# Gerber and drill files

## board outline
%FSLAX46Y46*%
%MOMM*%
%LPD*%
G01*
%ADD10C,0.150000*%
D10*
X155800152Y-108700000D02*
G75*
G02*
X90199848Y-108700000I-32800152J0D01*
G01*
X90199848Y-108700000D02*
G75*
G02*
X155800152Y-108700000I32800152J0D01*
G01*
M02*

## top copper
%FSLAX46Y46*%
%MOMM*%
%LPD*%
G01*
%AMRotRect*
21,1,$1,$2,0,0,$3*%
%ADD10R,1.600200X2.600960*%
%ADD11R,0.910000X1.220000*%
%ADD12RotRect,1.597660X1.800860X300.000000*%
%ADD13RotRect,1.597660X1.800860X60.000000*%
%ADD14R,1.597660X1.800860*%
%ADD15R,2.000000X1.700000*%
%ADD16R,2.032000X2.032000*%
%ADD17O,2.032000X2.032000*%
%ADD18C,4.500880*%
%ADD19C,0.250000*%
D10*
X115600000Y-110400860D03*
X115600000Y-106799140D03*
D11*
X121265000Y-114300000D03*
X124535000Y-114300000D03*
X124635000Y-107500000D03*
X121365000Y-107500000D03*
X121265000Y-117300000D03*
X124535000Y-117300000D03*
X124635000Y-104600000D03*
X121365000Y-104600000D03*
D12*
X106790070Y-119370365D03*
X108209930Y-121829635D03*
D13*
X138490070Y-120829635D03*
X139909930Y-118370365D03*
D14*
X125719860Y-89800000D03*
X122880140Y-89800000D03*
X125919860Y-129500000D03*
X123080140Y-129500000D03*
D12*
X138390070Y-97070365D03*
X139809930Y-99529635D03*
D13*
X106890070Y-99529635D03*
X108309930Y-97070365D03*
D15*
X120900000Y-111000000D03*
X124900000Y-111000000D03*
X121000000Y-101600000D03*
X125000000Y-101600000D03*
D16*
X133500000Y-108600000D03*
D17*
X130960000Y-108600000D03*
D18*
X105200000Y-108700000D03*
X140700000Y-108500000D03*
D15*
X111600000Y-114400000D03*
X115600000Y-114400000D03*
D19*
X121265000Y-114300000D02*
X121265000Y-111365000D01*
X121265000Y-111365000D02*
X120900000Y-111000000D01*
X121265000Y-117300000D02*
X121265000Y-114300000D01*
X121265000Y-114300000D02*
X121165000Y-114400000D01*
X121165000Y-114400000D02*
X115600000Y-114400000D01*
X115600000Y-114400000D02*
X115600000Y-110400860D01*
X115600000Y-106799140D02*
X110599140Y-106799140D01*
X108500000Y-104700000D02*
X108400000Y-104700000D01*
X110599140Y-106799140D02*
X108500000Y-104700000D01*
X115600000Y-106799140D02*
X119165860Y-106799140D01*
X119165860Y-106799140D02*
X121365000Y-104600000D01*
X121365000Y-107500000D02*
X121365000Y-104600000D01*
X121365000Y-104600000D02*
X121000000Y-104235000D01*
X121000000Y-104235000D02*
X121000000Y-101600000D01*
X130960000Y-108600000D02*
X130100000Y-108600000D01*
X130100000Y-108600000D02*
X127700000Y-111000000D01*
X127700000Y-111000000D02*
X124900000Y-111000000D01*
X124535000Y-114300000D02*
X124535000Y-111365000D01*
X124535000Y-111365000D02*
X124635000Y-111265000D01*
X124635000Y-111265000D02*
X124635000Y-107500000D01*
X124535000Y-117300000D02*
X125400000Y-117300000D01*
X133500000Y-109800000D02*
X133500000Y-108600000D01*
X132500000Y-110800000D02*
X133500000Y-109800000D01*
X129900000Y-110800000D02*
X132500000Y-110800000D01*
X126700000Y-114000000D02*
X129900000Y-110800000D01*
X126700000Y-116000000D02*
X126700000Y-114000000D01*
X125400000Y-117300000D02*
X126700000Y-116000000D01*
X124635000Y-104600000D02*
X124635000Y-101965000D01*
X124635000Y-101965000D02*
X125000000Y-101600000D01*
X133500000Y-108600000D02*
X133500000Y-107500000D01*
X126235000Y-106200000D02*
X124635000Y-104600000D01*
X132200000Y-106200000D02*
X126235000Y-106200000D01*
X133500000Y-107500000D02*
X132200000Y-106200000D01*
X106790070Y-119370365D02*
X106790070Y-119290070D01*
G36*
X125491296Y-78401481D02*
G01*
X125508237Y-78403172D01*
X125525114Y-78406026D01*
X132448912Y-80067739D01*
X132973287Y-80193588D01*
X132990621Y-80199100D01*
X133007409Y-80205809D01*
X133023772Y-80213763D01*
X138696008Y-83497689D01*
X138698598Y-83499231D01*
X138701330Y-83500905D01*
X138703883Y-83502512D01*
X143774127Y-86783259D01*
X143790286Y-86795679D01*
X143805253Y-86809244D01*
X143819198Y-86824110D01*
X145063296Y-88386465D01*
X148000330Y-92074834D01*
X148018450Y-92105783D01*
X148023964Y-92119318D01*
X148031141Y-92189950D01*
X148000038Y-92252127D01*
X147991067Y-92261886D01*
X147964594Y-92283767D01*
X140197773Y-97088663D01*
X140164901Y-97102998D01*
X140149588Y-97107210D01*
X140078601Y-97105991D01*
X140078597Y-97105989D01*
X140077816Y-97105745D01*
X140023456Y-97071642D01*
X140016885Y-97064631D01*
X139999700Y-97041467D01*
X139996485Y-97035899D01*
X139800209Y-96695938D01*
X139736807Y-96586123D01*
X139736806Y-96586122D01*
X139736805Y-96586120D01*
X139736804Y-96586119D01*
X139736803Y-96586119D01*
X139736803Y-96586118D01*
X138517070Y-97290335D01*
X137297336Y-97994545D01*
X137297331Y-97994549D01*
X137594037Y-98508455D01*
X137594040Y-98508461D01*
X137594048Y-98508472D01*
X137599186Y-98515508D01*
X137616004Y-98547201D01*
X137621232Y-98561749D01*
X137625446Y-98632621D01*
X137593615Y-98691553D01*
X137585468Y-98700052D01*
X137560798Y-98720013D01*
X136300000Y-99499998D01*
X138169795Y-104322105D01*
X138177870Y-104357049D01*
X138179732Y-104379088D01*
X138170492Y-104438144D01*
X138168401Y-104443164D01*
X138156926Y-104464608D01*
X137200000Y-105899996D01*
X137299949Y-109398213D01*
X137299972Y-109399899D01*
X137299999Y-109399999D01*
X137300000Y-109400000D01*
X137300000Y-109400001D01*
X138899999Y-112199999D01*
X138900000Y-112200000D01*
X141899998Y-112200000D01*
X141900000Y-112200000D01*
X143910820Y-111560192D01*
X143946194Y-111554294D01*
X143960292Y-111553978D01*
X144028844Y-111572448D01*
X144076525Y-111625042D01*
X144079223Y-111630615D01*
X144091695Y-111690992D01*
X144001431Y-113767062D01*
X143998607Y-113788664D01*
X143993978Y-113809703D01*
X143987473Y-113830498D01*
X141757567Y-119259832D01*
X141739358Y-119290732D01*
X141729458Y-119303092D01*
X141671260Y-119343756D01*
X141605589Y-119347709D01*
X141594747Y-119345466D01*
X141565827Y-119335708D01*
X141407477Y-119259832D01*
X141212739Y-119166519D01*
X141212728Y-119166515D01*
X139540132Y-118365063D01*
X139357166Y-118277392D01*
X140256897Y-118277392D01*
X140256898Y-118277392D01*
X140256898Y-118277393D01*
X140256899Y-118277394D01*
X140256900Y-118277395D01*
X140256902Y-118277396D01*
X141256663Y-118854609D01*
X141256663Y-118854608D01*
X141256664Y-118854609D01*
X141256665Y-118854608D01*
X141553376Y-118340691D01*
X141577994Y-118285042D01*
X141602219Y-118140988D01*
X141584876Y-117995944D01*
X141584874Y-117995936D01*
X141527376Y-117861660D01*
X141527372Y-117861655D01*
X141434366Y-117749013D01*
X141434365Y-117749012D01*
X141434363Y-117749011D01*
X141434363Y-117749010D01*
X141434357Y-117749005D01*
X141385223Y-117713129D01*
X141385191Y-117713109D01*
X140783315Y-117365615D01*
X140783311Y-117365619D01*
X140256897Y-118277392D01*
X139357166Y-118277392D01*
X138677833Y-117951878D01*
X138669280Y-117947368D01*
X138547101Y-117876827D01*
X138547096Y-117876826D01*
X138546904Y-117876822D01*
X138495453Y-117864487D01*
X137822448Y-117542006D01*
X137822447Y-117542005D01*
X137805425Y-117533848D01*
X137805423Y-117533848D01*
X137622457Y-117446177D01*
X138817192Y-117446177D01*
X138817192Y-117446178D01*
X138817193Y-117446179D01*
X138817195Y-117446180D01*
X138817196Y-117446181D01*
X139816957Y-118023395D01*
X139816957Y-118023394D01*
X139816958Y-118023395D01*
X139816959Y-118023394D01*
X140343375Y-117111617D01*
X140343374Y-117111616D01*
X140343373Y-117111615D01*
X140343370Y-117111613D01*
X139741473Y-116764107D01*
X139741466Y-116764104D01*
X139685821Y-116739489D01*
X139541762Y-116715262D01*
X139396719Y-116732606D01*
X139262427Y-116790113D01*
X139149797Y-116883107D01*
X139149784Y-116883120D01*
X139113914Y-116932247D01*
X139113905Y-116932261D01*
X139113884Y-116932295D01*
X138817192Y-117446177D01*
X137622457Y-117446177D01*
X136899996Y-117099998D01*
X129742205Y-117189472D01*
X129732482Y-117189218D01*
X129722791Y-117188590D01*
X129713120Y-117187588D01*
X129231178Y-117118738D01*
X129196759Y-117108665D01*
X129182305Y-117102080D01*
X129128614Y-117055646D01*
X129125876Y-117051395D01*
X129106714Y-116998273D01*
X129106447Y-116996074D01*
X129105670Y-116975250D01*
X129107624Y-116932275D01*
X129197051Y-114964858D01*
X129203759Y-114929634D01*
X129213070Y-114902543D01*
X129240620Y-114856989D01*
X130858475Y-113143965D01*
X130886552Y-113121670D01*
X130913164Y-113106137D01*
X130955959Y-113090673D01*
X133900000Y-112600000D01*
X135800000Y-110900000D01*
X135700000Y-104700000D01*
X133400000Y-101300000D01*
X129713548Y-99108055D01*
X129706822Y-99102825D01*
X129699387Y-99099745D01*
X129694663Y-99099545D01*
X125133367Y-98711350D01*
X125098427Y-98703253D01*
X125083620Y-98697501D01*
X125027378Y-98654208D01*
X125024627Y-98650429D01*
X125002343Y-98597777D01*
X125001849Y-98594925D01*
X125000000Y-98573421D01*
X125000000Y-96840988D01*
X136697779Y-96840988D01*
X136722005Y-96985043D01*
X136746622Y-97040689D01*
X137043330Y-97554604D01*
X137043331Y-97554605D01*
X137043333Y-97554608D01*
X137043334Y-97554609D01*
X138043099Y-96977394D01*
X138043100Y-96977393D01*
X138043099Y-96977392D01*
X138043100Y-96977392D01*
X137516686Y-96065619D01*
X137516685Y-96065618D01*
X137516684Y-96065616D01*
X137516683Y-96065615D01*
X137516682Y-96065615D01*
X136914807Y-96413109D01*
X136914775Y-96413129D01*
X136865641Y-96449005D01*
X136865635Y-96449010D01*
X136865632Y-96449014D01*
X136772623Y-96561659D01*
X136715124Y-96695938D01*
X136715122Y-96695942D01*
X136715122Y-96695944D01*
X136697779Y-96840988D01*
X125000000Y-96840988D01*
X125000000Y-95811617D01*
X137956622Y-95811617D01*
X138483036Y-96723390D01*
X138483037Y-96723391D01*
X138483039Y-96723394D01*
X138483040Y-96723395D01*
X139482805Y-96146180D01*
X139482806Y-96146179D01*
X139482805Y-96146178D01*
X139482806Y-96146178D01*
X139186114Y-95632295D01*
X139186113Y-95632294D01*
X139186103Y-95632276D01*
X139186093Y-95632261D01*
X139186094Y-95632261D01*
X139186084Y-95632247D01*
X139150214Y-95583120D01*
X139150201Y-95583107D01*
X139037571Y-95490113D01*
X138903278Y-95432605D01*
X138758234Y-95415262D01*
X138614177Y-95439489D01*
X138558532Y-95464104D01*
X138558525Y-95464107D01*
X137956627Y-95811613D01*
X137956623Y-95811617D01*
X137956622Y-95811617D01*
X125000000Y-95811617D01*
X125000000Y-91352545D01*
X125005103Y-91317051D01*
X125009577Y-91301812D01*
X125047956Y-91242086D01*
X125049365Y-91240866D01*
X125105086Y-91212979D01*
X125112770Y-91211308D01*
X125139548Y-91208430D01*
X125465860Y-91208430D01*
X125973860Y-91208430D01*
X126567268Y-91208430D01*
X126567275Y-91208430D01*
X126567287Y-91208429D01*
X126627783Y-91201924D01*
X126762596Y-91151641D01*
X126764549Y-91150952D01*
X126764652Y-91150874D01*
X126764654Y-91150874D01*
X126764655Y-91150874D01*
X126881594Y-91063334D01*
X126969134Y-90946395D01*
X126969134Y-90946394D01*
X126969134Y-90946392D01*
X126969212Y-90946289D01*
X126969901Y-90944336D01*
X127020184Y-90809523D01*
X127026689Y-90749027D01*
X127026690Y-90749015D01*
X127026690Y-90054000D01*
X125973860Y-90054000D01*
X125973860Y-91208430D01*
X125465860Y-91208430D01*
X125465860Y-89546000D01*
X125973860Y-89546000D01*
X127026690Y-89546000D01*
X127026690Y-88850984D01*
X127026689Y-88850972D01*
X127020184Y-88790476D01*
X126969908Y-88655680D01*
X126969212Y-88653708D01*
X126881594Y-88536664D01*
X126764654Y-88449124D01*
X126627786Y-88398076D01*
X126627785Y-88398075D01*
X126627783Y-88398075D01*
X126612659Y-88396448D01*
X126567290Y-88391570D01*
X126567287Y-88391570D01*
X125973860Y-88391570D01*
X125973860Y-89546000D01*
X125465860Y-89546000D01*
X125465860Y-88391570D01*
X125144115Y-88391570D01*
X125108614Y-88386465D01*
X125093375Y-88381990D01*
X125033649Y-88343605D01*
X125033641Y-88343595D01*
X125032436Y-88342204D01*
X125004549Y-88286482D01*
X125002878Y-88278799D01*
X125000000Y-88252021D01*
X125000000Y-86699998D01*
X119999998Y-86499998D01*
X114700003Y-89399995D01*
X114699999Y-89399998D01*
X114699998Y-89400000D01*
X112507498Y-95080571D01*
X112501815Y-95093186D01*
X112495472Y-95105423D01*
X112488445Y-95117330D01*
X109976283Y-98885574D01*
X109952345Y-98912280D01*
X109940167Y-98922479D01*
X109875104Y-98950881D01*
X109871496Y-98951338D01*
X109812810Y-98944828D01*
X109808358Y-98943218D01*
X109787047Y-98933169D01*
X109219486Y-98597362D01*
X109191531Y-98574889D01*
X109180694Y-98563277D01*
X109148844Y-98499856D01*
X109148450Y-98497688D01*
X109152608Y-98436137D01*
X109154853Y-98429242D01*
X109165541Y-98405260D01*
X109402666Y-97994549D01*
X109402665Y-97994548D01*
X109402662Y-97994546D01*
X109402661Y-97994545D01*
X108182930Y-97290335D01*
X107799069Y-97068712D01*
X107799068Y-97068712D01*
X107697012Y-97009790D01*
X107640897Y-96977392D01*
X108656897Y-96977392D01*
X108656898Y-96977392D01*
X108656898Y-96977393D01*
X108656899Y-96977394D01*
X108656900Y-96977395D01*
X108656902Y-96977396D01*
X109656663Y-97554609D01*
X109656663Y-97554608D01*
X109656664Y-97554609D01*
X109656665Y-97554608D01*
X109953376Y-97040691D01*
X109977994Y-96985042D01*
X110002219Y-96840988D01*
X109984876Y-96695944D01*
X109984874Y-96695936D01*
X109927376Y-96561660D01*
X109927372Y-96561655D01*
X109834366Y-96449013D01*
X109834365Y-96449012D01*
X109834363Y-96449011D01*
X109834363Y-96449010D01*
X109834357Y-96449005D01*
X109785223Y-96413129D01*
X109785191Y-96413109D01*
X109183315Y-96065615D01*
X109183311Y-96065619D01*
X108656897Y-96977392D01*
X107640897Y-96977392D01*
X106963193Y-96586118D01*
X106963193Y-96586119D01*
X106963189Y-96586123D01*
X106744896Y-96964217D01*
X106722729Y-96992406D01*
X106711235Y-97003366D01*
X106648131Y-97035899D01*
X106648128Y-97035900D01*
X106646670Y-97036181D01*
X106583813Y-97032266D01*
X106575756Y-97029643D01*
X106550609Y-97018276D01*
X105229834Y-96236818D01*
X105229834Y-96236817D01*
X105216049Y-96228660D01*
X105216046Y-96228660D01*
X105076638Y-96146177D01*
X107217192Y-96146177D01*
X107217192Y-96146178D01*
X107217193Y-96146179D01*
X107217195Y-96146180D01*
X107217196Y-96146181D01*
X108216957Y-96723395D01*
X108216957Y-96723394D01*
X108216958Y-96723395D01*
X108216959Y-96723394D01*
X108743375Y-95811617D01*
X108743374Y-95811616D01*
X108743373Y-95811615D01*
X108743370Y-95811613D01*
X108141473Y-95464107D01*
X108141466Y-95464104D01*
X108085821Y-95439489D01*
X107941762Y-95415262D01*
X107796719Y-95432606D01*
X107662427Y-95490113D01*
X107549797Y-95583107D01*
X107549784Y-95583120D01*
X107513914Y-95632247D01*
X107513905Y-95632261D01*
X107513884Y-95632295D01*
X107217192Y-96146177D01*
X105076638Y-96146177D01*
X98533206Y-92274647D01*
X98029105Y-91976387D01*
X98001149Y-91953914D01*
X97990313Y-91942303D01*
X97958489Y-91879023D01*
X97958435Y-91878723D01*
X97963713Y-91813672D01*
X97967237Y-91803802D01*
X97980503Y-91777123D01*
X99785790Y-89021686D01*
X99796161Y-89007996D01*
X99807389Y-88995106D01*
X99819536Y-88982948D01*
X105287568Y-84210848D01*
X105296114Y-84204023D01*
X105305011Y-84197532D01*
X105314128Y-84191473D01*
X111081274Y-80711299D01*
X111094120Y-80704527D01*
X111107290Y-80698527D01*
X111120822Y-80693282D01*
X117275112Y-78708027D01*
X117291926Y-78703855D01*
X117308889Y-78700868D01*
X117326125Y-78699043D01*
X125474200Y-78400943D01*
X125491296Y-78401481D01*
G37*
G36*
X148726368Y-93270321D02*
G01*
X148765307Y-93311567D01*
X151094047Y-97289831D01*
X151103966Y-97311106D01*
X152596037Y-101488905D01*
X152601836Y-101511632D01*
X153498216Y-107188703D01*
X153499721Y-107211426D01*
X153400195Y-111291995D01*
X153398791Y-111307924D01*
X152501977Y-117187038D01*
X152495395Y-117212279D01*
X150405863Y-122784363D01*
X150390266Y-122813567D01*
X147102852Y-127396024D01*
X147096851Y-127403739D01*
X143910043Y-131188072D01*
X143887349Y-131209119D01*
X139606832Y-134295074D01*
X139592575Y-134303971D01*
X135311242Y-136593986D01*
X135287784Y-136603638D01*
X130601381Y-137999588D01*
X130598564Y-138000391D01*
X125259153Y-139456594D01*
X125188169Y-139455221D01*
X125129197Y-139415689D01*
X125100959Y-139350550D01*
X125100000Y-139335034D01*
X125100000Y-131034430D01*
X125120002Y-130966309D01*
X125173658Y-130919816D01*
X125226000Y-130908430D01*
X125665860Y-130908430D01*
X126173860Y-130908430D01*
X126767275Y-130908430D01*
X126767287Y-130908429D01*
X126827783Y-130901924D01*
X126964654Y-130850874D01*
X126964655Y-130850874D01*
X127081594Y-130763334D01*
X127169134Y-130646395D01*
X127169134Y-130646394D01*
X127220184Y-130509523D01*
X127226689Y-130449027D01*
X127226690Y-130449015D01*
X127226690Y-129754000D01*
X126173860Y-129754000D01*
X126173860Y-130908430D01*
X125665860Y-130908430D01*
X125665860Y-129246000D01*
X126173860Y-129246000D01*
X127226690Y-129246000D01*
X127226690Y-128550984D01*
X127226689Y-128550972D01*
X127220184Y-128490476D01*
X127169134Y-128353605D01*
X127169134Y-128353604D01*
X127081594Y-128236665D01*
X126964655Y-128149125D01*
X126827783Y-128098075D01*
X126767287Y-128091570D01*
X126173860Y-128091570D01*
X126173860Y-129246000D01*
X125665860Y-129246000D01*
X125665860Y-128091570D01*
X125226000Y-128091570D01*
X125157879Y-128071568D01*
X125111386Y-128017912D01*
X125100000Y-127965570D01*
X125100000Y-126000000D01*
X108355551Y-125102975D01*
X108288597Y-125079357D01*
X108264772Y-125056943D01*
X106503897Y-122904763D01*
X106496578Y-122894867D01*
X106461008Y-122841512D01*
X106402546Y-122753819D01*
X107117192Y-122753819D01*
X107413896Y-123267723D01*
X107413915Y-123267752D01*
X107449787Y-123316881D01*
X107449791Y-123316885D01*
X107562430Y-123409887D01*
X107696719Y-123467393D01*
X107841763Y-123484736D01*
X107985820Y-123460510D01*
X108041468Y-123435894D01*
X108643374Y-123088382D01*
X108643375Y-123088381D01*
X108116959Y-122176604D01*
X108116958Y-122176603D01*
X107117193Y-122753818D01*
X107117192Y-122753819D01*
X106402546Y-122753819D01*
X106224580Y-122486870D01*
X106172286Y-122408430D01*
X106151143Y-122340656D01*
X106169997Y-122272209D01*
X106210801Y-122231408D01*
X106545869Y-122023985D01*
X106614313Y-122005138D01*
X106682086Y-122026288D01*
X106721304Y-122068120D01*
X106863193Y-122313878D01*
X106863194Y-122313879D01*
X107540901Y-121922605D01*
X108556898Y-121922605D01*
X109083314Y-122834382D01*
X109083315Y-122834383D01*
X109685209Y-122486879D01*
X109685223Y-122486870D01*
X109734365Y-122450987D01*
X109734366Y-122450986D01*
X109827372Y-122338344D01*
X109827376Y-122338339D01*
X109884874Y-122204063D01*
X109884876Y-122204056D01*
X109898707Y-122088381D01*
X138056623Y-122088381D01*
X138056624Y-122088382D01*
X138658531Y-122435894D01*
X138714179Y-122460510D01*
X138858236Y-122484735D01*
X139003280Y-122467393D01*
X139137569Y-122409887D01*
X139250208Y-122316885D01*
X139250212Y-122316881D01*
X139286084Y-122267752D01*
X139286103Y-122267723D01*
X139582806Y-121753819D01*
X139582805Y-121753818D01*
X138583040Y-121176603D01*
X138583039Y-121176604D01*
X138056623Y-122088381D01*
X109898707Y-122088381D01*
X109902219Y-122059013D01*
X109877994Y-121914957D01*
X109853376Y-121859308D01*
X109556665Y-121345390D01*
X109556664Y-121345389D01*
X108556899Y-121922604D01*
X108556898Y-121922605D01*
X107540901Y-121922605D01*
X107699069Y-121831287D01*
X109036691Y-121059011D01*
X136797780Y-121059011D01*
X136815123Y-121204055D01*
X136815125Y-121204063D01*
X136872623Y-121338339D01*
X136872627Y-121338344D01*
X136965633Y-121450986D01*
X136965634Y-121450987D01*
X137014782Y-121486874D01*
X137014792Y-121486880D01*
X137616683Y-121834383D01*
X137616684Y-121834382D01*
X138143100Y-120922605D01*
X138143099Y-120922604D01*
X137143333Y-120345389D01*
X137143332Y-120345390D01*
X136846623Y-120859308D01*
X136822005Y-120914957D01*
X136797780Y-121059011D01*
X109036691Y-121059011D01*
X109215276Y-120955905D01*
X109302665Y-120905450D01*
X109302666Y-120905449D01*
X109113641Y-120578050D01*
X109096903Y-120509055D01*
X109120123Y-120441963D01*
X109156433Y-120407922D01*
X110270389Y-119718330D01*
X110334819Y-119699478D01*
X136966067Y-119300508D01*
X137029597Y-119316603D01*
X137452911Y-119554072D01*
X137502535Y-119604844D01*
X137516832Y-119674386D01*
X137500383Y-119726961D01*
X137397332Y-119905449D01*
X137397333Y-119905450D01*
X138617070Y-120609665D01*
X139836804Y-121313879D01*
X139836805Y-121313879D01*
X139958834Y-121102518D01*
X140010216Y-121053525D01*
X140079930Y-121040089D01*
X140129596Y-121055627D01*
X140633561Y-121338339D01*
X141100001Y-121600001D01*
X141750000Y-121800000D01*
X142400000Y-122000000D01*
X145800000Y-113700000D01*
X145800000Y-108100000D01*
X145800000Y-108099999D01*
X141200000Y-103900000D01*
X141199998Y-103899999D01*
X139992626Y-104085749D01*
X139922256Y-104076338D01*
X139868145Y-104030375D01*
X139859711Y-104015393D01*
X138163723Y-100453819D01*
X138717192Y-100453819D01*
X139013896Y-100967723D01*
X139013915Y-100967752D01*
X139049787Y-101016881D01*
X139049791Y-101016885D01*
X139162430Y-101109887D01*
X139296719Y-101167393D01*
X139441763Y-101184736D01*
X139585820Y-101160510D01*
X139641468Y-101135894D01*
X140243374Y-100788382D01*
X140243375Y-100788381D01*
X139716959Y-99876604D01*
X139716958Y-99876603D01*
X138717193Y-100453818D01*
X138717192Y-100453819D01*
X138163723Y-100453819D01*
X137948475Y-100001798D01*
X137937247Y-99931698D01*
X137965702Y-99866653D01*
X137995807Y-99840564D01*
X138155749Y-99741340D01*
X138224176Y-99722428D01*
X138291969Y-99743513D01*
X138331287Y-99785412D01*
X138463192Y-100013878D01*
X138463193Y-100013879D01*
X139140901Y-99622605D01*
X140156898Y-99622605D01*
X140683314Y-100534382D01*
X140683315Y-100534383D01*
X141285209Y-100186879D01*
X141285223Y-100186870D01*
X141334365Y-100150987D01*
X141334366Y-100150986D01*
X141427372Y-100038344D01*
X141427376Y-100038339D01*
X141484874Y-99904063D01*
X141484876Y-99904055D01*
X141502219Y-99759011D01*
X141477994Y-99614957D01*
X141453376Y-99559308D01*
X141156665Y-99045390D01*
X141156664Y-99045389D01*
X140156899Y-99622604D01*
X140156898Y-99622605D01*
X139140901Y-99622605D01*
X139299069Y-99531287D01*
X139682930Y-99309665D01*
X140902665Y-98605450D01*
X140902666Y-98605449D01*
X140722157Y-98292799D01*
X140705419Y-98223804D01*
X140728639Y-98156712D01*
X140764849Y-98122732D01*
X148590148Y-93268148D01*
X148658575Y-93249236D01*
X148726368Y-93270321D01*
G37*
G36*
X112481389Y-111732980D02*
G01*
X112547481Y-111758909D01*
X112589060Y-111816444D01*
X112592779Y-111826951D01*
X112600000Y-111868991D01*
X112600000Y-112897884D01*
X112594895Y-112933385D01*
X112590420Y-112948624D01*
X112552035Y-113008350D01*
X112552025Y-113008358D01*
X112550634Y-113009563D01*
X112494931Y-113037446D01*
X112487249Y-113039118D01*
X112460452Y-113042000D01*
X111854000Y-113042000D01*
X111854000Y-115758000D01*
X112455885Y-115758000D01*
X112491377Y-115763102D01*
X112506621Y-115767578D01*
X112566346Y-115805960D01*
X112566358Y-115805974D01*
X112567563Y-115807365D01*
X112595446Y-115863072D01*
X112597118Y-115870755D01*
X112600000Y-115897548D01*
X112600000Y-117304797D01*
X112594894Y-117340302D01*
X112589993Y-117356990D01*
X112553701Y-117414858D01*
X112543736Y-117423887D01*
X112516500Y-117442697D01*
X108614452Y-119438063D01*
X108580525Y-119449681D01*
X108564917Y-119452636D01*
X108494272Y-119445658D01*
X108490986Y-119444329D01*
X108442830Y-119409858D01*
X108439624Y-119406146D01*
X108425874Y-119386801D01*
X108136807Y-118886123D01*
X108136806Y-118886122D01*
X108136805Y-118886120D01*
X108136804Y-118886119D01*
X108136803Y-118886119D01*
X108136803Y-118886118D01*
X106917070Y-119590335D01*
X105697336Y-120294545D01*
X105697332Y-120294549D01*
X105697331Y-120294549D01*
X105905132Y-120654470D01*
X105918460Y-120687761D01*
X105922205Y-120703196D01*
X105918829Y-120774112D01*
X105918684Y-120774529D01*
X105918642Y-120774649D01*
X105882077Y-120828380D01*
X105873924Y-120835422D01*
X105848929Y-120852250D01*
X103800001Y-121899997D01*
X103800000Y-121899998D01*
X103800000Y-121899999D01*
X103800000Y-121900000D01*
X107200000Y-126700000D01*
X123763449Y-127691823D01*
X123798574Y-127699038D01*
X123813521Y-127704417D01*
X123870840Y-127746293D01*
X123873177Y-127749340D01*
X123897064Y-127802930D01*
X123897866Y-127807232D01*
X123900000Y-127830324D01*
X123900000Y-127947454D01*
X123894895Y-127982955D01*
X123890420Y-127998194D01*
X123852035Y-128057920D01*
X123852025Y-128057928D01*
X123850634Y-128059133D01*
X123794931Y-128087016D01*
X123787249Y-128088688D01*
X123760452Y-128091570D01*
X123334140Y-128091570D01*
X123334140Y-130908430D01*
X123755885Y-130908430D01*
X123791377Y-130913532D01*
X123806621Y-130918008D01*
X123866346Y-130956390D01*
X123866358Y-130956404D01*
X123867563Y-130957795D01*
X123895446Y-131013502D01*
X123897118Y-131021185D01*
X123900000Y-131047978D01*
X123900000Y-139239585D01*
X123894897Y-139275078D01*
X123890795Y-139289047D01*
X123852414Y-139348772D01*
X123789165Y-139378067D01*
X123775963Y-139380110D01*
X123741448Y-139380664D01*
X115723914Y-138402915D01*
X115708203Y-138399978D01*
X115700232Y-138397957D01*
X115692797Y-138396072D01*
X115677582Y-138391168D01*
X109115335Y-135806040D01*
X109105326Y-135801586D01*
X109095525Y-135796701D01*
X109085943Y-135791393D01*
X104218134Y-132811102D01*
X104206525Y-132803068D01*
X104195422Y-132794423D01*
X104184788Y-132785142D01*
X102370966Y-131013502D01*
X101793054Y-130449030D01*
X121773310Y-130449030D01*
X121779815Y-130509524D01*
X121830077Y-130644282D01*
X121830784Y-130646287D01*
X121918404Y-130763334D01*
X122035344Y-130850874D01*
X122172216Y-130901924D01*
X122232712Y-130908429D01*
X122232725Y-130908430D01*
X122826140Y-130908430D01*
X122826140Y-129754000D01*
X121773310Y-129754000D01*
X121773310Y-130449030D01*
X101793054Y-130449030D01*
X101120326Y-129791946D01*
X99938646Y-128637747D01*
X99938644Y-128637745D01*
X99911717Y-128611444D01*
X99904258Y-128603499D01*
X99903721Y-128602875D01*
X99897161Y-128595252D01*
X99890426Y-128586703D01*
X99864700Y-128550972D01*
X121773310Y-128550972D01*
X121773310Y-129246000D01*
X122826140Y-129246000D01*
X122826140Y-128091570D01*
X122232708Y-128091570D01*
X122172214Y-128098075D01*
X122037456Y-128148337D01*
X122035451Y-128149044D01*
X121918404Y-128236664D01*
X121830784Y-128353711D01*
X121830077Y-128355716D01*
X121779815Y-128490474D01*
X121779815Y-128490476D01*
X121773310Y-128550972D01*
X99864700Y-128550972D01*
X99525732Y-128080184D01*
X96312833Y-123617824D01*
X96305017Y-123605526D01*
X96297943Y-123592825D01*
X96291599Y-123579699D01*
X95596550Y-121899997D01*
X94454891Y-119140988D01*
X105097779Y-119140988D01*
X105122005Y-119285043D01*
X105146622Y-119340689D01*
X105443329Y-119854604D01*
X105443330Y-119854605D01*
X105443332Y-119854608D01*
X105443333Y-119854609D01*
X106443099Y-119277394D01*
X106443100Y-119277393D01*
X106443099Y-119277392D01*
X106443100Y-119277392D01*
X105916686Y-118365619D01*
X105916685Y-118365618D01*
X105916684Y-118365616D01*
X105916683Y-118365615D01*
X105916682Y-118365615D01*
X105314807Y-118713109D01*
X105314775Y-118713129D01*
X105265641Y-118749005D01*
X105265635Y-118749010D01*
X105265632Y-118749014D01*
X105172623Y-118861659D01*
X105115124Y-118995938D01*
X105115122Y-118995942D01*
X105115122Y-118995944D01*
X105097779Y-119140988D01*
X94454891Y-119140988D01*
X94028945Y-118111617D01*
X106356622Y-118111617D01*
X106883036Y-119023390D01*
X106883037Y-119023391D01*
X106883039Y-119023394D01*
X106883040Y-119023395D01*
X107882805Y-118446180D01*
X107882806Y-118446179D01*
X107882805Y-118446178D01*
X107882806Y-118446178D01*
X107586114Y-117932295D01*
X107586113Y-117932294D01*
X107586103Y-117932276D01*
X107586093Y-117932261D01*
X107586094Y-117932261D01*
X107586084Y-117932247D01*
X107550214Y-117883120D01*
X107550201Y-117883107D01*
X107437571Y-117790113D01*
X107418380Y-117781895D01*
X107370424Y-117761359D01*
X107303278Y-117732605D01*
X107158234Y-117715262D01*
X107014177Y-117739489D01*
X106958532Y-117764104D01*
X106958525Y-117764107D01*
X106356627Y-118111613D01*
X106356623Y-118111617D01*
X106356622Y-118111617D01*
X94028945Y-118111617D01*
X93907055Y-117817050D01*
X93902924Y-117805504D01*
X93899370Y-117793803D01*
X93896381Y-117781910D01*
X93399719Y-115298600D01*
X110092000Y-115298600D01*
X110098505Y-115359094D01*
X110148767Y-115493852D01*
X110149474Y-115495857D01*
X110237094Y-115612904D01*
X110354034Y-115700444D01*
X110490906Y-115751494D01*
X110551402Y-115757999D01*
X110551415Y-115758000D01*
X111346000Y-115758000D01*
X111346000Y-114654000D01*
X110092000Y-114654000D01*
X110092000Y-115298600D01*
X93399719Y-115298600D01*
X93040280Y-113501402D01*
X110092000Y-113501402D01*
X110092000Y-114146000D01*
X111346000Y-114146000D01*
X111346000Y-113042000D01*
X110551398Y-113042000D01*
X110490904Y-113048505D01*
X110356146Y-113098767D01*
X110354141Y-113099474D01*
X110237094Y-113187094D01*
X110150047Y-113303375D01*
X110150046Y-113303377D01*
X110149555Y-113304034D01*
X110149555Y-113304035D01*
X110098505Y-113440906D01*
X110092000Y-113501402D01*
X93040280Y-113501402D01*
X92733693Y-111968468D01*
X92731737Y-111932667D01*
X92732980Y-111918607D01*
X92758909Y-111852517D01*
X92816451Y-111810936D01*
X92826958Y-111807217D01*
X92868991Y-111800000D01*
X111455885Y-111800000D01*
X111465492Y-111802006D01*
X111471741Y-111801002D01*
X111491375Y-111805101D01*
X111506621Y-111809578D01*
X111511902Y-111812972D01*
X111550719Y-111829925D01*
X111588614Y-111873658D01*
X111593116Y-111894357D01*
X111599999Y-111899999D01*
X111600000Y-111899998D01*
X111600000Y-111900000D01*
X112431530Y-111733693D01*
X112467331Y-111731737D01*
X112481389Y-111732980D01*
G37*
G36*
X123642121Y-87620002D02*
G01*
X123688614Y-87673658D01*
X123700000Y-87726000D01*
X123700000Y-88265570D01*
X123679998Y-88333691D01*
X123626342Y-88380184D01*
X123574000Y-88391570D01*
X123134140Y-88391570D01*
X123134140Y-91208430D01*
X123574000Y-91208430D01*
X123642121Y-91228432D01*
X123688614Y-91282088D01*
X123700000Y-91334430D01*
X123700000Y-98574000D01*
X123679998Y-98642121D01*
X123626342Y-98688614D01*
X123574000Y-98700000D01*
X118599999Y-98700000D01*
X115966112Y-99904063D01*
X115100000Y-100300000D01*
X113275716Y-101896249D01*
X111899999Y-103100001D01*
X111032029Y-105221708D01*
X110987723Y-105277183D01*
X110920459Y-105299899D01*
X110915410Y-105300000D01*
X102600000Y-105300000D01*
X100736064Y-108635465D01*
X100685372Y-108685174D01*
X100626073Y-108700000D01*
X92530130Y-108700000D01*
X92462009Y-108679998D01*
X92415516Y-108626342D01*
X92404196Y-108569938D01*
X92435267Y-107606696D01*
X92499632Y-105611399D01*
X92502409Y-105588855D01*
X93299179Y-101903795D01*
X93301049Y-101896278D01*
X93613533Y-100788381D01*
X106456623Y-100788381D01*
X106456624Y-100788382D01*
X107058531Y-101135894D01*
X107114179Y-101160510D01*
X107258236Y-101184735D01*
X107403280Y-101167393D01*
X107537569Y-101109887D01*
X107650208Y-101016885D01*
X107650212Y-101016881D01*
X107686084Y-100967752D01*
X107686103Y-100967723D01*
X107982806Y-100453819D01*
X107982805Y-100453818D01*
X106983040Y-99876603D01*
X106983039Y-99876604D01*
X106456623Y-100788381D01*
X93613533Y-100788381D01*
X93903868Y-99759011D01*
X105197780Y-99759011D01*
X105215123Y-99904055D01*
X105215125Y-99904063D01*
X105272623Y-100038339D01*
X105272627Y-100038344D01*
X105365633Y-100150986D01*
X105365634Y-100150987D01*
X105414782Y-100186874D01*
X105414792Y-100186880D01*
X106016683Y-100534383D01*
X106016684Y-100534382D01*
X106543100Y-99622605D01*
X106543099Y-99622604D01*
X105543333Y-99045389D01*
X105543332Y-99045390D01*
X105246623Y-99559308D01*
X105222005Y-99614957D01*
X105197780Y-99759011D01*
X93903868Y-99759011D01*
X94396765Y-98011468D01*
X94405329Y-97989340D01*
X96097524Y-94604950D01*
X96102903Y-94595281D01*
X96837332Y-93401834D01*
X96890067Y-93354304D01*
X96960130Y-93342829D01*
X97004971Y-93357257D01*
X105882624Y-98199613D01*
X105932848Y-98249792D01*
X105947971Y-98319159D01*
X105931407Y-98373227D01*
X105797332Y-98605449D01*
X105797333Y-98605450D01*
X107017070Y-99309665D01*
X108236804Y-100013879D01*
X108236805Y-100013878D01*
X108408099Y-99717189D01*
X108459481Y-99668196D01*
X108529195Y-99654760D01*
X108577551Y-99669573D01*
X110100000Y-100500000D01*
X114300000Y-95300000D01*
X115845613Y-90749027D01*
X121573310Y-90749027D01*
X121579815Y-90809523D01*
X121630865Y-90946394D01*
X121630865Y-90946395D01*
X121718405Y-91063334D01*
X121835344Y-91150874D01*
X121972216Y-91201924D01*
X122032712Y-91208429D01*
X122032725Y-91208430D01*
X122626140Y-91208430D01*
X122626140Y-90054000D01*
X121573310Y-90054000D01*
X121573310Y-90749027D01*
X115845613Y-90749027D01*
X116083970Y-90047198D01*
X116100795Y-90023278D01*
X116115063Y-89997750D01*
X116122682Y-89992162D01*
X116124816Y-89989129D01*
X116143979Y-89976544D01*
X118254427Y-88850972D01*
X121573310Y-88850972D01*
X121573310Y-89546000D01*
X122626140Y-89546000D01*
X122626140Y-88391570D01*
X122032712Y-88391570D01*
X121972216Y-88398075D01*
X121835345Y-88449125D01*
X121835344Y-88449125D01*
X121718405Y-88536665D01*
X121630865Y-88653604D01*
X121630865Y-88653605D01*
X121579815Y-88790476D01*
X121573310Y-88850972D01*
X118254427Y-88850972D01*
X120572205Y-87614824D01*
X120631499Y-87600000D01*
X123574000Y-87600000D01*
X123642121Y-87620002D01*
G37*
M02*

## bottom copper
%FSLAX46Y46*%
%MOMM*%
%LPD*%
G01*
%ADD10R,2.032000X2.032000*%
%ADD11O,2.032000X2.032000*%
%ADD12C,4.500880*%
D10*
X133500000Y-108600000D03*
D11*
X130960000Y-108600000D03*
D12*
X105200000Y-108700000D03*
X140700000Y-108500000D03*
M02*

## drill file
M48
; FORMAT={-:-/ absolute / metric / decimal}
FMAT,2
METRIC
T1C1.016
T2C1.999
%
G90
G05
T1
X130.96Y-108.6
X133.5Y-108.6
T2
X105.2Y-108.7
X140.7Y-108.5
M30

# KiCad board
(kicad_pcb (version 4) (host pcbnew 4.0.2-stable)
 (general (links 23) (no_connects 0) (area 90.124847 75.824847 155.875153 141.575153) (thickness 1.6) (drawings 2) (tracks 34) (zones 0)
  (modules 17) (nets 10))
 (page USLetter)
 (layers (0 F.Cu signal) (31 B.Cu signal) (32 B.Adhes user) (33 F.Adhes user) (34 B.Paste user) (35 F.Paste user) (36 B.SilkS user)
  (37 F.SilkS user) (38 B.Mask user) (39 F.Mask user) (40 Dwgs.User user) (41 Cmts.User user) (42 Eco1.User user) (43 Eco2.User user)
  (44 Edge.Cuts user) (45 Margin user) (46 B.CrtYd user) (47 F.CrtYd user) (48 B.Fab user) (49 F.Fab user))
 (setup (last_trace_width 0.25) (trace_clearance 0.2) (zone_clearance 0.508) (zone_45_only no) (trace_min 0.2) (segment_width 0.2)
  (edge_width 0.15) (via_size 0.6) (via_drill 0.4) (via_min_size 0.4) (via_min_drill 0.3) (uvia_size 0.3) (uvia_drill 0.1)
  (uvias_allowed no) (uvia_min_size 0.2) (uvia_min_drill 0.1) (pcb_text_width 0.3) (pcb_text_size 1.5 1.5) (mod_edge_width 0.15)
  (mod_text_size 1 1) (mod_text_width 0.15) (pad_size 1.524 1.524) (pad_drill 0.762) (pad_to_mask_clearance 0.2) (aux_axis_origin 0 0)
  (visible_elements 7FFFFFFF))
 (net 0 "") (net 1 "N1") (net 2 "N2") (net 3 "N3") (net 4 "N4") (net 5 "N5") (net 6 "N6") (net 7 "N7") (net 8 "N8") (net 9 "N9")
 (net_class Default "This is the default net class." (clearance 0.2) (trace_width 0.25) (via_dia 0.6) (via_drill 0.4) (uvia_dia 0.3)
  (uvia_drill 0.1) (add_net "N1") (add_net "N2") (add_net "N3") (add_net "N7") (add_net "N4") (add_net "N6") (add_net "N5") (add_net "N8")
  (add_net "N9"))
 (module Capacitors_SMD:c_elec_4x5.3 (layer F.Cu) (at 115.6 108.6 270)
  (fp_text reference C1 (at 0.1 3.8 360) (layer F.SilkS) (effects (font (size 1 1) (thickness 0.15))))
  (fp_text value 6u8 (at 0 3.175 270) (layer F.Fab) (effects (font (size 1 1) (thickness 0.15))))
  (pad 1 smd rect (at 1.80086 0 270) (size 2.60096 1.6002) (layers F.Cu F.Paste F.Mask) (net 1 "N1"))
  (pad 2 smd rect (at -1.80086 0 270) (size 2.60096 1.6002) (layers F.Cu F.Paste F.Mask) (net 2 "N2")))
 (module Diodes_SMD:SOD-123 (layer F.Cu) (at 122.9 114.3)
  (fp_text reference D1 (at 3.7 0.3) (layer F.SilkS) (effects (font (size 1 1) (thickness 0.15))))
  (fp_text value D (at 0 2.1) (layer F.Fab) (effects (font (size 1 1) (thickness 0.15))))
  (pad 1 smd rect (at -1.635 0) (size 0.91 1.22) (layers F.Cu F.Paste F.Mask) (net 1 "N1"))
  (pad 2 smd rect (at 1.635 0) (size 0.91 1.22) (layers F.Cu F.Paste F.Mask) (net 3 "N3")))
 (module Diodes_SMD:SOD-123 (layer F.Cu) (at 123 107.5 180)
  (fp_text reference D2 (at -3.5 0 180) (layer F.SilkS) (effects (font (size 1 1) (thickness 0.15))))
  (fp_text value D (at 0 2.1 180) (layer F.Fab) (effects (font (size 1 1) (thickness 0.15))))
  (pad 1 smd rect (at -1.635 0 180) (size 0.91 1.22) (layers F.Cu F.Paste F.Mask) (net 3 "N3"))
  (pad 2 smd rect (at 1.635 0 180) (size 0.91 1.22) (layers F.Cu F.Paste F.Mask) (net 2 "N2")))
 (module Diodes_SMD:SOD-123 (layer F.Cu) (at 122.9 117.3)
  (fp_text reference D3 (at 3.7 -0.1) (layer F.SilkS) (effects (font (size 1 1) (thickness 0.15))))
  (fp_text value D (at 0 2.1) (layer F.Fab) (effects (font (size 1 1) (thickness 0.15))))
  (pad 1 smd rect (at -1.635 0) (size 0.91 1.22) (layers F.Cu F.Paste F.Mask) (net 1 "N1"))
  (pad 2 smd rect (at 1.635 0) (size 0.91 1.22) (layers F.Cu F.Paste F.Mask) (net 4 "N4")))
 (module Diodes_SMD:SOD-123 (layer F.Cu) (at 123 104.6 180)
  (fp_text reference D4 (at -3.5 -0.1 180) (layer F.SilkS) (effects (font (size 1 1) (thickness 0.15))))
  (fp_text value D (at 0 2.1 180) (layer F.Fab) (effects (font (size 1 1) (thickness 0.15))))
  (pad 1 smd rect (at -1.635 0 180) (size 0.91 1.22) (layers F.Cu F.Paste F.Mask) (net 4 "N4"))
  (pad 2 smd rect (at 1.635 0 180) (size 0.91 1.22) (layers F.Cu F.Paste F.Mask) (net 2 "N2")))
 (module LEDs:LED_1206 (layer F.Cu) (at 107.5 120.6 120)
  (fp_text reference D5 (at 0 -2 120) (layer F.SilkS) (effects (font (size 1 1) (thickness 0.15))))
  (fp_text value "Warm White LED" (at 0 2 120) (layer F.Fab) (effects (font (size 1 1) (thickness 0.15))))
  (pad 2 smd rect (at 1.41986 0 300) (size 1.59766 1.80086) (layers F.Cu F.Paste F.Mask) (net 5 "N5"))
  (pad 1 smd rect (at -1.41986 0 300) (size 1.59766 1.80086) (layers F.Cu F.Paste F.Mask) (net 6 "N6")))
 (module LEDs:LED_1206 (layer F.Cu) (at 139.2 119.6 240)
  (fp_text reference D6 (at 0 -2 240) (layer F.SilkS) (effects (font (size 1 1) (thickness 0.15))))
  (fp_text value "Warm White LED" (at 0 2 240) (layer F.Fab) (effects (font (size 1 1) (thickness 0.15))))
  (pad 2 smd rect (at 1.41986 0 60) (size 1.59766 1.80086) (layers F.Cu F.Paste F.Mask) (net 6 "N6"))
  (pad 1 smd rect (at -1.41986 0 60) (size 1.59766 1.80086) (layers F.Cu F.Paste F.Mask) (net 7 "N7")))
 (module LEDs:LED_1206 (layer F.Cu) (at 124.3 89.8)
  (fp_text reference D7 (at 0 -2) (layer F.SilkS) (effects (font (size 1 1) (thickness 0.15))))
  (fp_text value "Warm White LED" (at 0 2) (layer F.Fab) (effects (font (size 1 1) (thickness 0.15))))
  (pad 2 smd rect (at 1.41986 0 180) (size 1.59766 1.80086) (layers F.Cu F.Paste F.Mask) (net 7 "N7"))
  (pad 1 smd rect (at -1.41986 0 180) (size 1.59766 1.80086) (layers F.Cu F.Paste F.Mask) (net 2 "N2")))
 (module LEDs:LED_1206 (layer F.Cu) (at 124.5 129.5)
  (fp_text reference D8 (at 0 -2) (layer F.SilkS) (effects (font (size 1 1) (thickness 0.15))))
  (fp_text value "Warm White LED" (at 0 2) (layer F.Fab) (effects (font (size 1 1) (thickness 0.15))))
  (pad 2 smd rect (at 1.41986 0 180) (size 1.59766 1.80086) (layers F.Cu F.Paste F.Mask) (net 6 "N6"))
  (pad 1 smd rect (at -1.41986 0 180) (size 1.59766 1.80086) (layers F.Cu F.Paste F.Mask) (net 5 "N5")))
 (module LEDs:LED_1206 (layer F.Cu) (at 139.1 98.3 120)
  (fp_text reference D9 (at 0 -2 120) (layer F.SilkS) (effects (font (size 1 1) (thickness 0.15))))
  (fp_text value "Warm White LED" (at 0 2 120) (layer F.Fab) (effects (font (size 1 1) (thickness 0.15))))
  (pad 2 smd rect (at 1.41986 0 300) (size 1.59766 1.80086) (layers F.Cu F.Paste F.Mask) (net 7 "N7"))
  (pad 1 smd rect (at -1.41986 0 300) (size 1.59766 1.80086) (layers F.Cu F.Paste F.Mask) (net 6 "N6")))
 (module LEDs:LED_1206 (layer F.Cu) (at 107.6 98.3 240)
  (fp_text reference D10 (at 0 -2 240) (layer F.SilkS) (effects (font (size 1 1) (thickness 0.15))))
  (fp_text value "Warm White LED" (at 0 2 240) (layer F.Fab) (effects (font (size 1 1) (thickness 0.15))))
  (pad 2 smd rect (at 1.41986 0 60) (size 1.59766 1.80086) (layers F.Cu F.Paste F.Mask) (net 2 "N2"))
  (pad 1 smd rect (at -1.41986 0 60) (size 1.59766 1.80086) (layers F.Cu F.Paste F.Mask) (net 7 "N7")))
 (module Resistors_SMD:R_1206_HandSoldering (layer F.Cu) (at 122.9 111)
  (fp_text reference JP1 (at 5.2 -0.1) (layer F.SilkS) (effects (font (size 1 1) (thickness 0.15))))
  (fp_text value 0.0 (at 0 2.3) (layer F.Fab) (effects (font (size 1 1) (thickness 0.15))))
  (pad 1 smd rect (at -2 0) (size 2 1.7) (layers F.Cu F.Paste F.Mask) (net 1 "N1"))
  (pad 2 smd rect (at 2 0) (size 2 1.7) (layers F.Cu F.Paste F.Mask) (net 3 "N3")))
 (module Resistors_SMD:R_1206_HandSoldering (layer F.Cu) (at 123 101.6)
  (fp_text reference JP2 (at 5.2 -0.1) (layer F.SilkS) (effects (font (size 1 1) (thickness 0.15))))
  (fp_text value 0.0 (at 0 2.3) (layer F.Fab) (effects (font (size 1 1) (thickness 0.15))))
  (pad 1 smd rect (at -2 0) (size 2 1.7) (layers F.Cu F.Paste F.Mask) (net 2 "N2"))
  (pad 2 smd rect (at 2 0) (size 2 1.7) (layers F.Cu F.Paste F.Mask) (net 4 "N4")))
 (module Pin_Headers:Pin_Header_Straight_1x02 (layer F.Cu) (at 133.5 108.6 270)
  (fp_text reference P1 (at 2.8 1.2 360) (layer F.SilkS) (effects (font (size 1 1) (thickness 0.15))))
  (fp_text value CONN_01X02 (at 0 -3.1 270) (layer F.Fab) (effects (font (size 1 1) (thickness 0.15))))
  (pad 1 thru_hole rect (at 0 0 270) (size 2.032 2.032) (drill 1.016) (layers *.Cu *.Mask F.SilkS) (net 4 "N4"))
  (pad 2 thru_hole oval (at 0 2.54 270) (size 2.032 2.032) (drill 1.016) (layers *.Cu *.Mask F.SilkS) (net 3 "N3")))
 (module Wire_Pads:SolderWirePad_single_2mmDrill (layer F.Cu) (at 105.2 108.7)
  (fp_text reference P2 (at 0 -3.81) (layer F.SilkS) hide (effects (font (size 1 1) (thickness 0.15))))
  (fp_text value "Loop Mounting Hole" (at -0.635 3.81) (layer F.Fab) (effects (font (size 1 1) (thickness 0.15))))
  (pad 1 thru_hole circle (at 0 0) (size 4.50088 4.50088) (drill 1.99898) (layers *.Cu *.Mask F.SilkS) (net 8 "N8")))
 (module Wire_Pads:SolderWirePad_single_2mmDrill (layer F.Cu) (at 140.7 108.5)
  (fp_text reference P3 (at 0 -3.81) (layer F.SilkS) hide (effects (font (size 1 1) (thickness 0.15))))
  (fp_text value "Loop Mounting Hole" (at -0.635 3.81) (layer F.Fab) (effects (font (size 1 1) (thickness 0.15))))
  (pad 1 thru_hole circle (at 0 0) (size 4.50088 4.50088) (drill 1.99898) (layers *.Cu *.Mask F.SilkS) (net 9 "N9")))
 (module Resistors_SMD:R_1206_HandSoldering (layer F.Cu) (at 113.6 114.4)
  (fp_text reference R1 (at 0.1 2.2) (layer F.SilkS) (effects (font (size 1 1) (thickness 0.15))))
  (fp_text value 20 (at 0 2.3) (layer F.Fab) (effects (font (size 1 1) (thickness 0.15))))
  (pad 1 smd rect (at -2 0) (size 2 1.7) (layers F.Cu F.Paste F.Mask) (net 5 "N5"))
  (pad 2 smd rect (at 2 0) (size 2 1.7) (layers F.Cu F.Paste F.Mask) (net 1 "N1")))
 (gr_circle (center 123 108.7) (end 155.8 108.8) (layer Edge.Cuts) (width 0.15))
 (segment (start 121.265 114.3) (end 121.265 111.365) (width 0.25) (layer F.Cu) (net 1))
 (segment (start 121.265 111.365) (end 120.9 111) (width 0.25) (layer F.Cu) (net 1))
 (segment (start 121.265 117.3) (end 121.265 114.3) (width 0.25) (layer F.Cu) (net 1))
 (segment (start 121.265 114.3) (end 121.165 114.4) (width 0.25) (layer F.Cu) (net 1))
 (segment (start 121.165 114.4) (end 115.6 114.4) (width 0.25) (layer F.Cu) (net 1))
 (segment (start 115.6 114.4) (end 115.6 110.40086) (width 0.25) (layer F.Cu) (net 1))
 (segment (start 115.6 106.79914) (end 110.59914 106.79914) (width 0.25) (layer F.Cu) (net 2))
 (segment (start 108.5 104.7) (end 108.4 104.7) (width 0.25) (layer F.Cu) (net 2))
 (segment (start 110.59914 106.79914) (end 108.5 104.7) (width 0.25) (layer F.Cu) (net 2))
 (segment (start 115.6 106.79914) (end 119.16586 106.79914) (width 0.25) (layer F.Cu) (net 2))
 (segment (start 119.16586 106.79914) (end 121.365 104.6) (width 0.25) (layer F.Cu) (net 2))
 (segment (start 121.365 107.5) (end 121.365 104.6) (width 0.25) (layer F.Cu) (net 2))
 (segment (start 121.365 104.6) (end 121 104.235) (width 0.25) (layer F.Cu) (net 2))
 (segment (start 121 104.235) (end 121 101.6) (width 0.25) (layer F.Cu) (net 2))
 (segment (start 130.96 108.6) (end 130.1 108.6) (width 0.25) (layer F.Cu) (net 3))
 (segment (start 130.1 108.6) (end 127.7 111) (width 0.25) (layer F.Cu) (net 3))
 (segment (start 127.7 111) (end 124.9 111) (width 0.25) (layer F.Cu) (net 3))
 (segment (start 124.535 114.3) (end 124.535 111.365) (width 0.25) (layer F.Cu) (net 3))
 (segment (start 124.535 111.365) (end 124.635 111.265) (width 0.25) (layer F.Cu) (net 3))
 (segment (start 124.635 111.265) (end 124.635 107.5) (width 0.25) (layer F.Cu) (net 3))
 (segment (start 124.535 117.3) (end 125.4 117.3) (width 0.25) (layer F.Cu) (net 4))
 (segment (start 133.5 109.8) (end 133.5 108.6) (width 0.25) (layer F.Cu) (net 4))
 (segment (start 132.5 110.8) (end 133.5 109.8) (width 0.25) (layer F.Cu) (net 4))
 (segment (start 129.9 110.8) (end 132.5 110.8) (width 0.25) (layer F.Cu) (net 4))
 (segment (start 126.7 114) (end 129.9 110.8) (width 0.25) (layer F.Cu) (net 4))
 (segment (start 126.7 116) (end 126.7 114) (width 0.25) (layer F.Cu) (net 4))
 (segment (start 125.4 117.3) (end 126.7 116) (width 0.25) (layer F.Cu) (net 4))
 (segment (start 124.635 104.6) (end 124.635 101.965) (width 0.25) (layer F.Cu) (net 4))
 (segment (start 124.635 101.965) (end 125 101.6) (width 0.25) (layer F.Cu) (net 4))
 (segment (start 133.5 108.6) (end 133.5 107.5) (width 0.25) (layer F.Cu) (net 4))
 (segment (start 126.235 106.2) (end 124.635 104.6) (width 0.25) (layer F.Cu) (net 4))
 (segment (start 132.2 106.2) (end 126.235 106.2) (width 0.25) (layer F.Cu) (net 4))
 (segment (start 133.5 107.5) (end 132.2 106.2) (width 0.25) (layer F.Cu) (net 4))
 (segment (start 106.79007 119.370365) (end 106.79007 119.29007) (width 0.25) (layer F.Cu) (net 5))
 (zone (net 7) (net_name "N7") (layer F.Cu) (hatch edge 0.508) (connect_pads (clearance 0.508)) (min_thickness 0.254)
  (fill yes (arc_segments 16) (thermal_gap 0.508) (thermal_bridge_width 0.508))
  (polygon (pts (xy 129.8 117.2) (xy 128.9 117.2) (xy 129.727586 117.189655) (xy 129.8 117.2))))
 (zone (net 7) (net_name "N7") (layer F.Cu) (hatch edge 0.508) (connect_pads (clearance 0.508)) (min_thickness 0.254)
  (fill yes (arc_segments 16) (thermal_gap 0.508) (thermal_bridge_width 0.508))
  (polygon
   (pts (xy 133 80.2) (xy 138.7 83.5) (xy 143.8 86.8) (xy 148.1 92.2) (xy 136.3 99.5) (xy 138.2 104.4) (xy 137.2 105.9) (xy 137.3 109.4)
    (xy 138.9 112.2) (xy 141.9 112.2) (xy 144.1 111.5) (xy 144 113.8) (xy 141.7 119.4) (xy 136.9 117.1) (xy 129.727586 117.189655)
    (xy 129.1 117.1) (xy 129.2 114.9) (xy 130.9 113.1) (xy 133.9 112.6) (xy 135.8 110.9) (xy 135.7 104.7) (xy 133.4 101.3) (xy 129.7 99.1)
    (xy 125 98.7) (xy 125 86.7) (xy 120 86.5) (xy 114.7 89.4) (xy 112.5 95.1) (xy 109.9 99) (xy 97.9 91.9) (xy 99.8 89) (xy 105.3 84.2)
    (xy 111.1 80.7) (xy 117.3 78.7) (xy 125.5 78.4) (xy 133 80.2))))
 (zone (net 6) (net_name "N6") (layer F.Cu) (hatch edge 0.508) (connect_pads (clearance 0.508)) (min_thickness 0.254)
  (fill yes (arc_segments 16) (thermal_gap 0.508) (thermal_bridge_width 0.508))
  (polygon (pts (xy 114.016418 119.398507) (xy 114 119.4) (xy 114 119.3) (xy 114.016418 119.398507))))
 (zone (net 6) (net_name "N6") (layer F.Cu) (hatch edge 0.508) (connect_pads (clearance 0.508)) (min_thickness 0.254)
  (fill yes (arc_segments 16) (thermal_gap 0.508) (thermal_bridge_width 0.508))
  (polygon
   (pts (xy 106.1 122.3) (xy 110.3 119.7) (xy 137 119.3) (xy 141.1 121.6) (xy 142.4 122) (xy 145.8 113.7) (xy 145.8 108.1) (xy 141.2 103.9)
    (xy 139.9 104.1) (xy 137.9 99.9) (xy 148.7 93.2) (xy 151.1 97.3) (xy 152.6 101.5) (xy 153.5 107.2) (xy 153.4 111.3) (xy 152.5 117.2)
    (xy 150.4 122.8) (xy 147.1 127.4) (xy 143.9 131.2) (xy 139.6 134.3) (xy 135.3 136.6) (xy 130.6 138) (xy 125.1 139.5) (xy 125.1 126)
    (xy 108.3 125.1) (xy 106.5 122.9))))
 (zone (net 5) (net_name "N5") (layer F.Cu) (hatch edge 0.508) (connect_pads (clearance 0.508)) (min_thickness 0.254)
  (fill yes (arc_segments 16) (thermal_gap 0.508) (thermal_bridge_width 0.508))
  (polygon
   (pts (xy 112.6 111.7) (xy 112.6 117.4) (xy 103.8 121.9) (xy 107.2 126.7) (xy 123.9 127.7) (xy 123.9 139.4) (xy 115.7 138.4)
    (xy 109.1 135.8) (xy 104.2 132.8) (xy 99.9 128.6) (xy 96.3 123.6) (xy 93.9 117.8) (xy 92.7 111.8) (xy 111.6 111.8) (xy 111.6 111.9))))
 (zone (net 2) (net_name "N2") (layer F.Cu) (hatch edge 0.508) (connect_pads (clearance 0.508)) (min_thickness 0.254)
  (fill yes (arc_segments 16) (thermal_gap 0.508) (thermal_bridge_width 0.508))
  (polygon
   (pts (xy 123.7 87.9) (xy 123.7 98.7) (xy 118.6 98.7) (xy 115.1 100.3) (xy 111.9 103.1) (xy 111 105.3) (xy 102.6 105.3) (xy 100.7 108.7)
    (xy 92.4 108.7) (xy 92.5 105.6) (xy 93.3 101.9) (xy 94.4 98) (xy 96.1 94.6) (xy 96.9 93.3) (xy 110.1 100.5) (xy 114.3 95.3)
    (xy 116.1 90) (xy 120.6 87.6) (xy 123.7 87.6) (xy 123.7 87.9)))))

